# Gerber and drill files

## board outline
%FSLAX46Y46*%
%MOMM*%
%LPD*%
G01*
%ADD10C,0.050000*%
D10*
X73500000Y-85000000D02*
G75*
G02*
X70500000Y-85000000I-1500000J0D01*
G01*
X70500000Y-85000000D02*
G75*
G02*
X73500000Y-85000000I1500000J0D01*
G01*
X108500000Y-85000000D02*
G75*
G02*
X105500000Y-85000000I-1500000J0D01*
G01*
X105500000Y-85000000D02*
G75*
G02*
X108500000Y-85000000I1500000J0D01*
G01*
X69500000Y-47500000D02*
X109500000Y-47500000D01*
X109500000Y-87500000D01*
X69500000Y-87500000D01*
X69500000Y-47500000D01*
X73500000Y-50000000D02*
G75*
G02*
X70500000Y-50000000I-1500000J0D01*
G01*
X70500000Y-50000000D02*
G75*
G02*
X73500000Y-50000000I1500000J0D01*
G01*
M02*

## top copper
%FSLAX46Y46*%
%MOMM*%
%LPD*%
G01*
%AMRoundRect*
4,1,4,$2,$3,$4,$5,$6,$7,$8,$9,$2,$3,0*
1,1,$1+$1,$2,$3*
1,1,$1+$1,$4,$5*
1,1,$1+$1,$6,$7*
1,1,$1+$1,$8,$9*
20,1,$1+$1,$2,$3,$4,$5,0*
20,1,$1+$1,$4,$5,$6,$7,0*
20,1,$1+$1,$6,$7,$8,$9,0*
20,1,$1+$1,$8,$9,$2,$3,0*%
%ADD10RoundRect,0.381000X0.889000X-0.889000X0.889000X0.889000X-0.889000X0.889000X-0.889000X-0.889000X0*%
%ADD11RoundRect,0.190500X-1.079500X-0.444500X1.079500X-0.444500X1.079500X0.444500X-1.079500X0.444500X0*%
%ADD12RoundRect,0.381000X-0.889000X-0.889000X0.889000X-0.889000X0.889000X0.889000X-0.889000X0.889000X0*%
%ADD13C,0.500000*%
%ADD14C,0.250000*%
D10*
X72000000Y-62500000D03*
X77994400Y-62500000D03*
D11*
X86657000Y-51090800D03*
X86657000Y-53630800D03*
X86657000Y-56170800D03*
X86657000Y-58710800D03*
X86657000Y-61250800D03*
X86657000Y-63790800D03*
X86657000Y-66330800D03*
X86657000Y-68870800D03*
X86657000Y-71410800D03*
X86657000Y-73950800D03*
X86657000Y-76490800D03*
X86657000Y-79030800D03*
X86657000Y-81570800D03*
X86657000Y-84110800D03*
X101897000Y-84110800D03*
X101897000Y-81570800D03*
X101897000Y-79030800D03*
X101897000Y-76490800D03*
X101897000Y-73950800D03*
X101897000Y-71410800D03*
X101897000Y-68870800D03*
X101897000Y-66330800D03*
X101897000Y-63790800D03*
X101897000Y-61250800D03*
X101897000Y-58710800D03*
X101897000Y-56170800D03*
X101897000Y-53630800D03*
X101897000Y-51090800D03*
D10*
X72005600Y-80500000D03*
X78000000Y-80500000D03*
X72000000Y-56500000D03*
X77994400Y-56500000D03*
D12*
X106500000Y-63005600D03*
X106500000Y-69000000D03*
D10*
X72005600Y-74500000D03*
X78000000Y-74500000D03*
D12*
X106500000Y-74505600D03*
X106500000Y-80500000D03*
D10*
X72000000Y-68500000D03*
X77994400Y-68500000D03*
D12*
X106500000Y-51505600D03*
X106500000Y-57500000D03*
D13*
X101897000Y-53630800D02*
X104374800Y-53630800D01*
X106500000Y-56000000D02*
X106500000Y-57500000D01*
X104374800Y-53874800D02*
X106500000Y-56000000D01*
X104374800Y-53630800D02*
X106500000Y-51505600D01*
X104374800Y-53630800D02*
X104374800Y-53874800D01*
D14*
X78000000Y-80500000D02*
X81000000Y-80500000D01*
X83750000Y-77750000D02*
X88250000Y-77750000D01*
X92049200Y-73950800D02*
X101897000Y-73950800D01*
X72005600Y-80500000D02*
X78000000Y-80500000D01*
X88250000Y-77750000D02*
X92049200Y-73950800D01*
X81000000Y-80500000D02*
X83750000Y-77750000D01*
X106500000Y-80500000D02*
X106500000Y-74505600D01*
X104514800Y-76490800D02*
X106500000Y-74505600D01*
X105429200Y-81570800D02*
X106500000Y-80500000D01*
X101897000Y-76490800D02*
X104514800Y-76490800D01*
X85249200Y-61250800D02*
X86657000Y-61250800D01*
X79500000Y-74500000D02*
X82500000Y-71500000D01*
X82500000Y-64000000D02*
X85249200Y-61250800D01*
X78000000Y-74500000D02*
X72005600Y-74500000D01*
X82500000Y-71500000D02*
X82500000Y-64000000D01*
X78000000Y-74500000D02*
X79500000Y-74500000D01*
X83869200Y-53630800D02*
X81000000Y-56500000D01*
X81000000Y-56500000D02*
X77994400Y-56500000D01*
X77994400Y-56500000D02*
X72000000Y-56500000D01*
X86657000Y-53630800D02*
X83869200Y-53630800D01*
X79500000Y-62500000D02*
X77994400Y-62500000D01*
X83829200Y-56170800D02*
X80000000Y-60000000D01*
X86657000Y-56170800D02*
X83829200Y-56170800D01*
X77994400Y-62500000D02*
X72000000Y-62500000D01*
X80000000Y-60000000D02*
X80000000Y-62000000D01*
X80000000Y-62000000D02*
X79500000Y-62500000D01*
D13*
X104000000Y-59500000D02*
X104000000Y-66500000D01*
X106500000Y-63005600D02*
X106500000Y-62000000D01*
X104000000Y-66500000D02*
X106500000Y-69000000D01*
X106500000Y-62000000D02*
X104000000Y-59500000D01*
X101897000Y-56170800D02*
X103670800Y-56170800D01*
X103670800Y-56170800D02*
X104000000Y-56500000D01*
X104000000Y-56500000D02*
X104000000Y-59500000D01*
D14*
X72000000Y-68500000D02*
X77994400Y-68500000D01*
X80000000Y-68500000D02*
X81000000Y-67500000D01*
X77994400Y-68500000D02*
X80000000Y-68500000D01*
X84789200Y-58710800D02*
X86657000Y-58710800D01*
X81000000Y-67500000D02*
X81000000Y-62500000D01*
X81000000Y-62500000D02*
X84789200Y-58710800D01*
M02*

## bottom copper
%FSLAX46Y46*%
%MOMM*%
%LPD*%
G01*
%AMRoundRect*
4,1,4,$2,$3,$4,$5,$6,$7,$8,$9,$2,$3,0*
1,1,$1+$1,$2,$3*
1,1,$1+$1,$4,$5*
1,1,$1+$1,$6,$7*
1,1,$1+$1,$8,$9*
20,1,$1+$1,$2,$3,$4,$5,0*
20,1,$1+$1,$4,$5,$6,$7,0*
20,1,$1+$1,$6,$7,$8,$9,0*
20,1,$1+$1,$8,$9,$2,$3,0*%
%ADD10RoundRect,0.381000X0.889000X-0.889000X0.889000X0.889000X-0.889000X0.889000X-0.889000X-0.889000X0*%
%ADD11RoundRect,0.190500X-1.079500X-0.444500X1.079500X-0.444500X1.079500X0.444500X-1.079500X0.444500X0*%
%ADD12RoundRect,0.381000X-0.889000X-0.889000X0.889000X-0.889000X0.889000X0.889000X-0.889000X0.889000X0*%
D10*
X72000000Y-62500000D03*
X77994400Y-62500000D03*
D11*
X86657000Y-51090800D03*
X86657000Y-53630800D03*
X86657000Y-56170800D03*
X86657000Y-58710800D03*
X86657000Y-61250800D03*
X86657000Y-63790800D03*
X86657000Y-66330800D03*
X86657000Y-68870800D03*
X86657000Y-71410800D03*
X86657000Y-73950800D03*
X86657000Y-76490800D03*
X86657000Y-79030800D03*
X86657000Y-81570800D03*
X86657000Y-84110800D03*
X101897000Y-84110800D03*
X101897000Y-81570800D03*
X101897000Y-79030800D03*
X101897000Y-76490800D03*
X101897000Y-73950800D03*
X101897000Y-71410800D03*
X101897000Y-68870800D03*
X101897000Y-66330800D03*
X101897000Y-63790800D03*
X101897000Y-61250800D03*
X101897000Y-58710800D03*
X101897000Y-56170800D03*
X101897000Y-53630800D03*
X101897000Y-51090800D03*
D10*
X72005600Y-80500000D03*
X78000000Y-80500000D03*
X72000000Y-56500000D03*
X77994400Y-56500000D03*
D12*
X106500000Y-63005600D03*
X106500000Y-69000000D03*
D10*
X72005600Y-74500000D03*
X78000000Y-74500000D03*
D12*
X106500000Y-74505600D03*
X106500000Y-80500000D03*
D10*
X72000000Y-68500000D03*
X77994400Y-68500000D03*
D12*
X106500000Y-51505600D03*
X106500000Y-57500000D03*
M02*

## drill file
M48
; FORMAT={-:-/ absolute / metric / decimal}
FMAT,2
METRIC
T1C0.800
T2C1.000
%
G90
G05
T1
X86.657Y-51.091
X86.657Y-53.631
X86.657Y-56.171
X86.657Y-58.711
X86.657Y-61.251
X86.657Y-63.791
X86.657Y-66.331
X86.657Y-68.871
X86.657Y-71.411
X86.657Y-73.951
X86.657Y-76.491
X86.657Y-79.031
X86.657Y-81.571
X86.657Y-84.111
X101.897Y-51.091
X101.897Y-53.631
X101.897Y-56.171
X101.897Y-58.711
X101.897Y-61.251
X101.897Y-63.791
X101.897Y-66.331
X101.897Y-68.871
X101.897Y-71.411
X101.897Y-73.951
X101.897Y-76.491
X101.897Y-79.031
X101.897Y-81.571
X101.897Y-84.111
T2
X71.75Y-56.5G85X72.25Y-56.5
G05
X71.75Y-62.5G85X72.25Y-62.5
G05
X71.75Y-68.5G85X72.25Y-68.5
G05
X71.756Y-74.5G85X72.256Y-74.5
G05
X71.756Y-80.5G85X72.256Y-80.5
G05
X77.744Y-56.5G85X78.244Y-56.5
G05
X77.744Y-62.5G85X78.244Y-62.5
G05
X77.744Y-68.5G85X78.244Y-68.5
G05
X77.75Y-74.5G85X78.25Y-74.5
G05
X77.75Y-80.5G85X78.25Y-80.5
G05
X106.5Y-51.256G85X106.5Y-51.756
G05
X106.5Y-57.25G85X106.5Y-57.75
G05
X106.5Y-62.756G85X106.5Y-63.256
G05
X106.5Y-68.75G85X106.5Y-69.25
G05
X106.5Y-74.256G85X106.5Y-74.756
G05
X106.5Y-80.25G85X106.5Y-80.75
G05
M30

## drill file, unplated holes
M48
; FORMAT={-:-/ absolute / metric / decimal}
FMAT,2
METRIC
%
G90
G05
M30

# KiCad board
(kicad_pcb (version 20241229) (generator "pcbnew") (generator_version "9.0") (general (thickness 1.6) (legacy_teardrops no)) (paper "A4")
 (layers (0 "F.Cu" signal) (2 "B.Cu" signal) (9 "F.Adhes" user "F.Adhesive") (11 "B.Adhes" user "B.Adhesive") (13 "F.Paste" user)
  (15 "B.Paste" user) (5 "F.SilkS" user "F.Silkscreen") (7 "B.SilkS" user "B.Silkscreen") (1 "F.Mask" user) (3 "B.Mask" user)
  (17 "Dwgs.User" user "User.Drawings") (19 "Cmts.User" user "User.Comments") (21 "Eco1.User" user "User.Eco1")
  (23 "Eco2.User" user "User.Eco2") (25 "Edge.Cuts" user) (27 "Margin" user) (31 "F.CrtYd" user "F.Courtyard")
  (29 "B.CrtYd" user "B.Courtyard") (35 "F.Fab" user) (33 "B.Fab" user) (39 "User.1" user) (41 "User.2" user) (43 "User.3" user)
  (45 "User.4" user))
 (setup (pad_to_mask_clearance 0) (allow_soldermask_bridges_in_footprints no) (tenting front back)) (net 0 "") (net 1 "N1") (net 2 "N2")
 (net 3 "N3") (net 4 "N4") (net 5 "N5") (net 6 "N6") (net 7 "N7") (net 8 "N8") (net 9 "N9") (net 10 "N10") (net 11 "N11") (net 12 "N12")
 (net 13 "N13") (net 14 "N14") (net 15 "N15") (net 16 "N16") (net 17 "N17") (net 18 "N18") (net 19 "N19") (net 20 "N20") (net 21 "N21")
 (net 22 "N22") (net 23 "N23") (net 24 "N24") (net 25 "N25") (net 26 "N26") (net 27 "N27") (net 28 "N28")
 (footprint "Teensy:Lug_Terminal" (layer "F.Cu") (at 75.2512 62.5 90)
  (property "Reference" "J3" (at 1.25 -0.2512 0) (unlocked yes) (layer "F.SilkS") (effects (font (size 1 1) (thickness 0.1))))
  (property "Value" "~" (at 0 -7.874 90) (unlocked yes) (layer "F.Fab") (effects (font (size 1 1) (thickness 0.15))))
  (pad "1" thru_hole roundrect (at 0 -3.2512 90) (size 2.54 2.54) (drill oval 1 1.5) (layers "*.Cu" "*.Mask") (remove_unused_layers no)
   (roundrect_rratio 0.15) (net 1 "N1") (thermal_bridge_angle 45))
  (pad "1" thru_hole roundrect (at 0 2.7432 90) (size 2.54 2.54) (drill oval 1 1.5) (layers "*.Cu" "*.Mask") (remove_unused_layers no)
   (roundrect_rratio 0.15) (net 1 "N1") (thermal_bridge_angle 45)))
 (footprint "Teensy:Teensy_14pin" (layer "F.Cu") (at 91.737 58.7108)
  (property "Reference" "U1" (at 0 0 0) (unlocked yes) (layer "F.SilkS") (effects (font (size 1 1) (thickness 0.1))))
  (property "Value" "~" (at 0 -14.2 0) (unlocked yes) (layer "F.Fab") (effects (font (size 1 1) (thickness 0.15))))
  (pad "1" thru_hole roundrect (at -5.08 -7.62) (size 2.54 1.27) (drill 0.8) (layers "*.Cu" "*.Mask") (remove_unused_layers no)
   (roundrect_rratio 0.15) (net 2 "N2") (thermal_bridge_angle 45))
  (pad "2" thru_hole roundrect (at -5.08 -5.08) (size 2.54 1.27) (drill 0.8) (layers "*.Cu" "*.Mask") (remove_unused_layers no)
   (roundrect_rratio 0.15) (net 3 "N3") (thermal_bridge_angle 45))
  (pad "3" thru_hole roundrect (at -5.08 -2.54) (size 2.54 1.27) (drill 0.8) (layers "*.Cu" "*.Mask") (remove_unused_layers no)
   (roundrect_rratio 0.15) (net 1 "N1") (thermal_bridge_angle 45))
  (pad "4" thru_hole roundrect (at -5.08 0) (size 2.54 1.27) (drill 0.8) (layers "*.Cu" "*.Mask") (remove_unused_layers no)
   (roundrect_rratio 0.15) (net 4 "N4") (thermal_bridge_angle 45))
  (pad "5" thru_hole roundrect (at -5.08 2.54) (size 2.54 1.27) (drill 0.8) (layers "*.Cu" "*.Mask") (remove_unused_layers no)
   (roundrect_rratio 0.15) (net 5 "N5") (thermal_bridge_angle 45))
  (pad "6" thru_hole roundrect (at -5.08 5.08) (size 2.54 1.27) (drill 0.8) (layers "*.Cu" "*.Mask") (remove_unused_layers no)
   (roundrect_rratio 0.15) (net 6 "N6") (thermal_bridge_angle 45))
  (pad "7" thru_hole roundrect (at -5.08 7.62) (size 2.54 1.27) (drill 0.8) (layers "*.Cu" "*.Mask") (remove_unused_layers no)
   (roundrect_rratio 0.15) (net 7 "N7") (thermal_bridge_angle 45))
  (pad "8" thru_hole roundrect (at -5.08 10.16) (size 2.54 1.27) (drill 0.8) (layers "*.Cu" "*.Mask") (remove_unused_layers no)
   (roundrect_rratio 0.15) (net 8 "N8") (thermal_bridge_angle 45))
  (pad "9" thru_hole roundrect (at -5.08 12.7) (size 2.54 1.27) (drill 0.8) (layers "*.Cu" "*.Mask") (remove_unused_layers no)
   (roundrect_rratio 0.15) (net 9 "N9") (thermal_bridge_angle 45))
  (pad "10" thru_hole roundrect (at -5.08 15.24) (size 2.54 1.27) (drill 0.8) (layers "*.Cu" "*.Mask") (remove_unused_layers no)
   (roundrect_rratio 0.15) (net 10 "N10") (thermal_bridge_angle 45))
  (pad "11" thru_hole roundrect (at -5.08 17.78) (size 2.54 1.27) (drill 0.8) (layers "*.Cu" "*.Mask") (remove_unused_layers no)
   (roundrect_rratio 0.15) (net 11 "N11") (thermal_bridge_angle 45))
  (pad "12" thru_hole roundrect (at -5.08 20.32) (size 2.54 1.27) (drill 0.8) (layers "*.Cu" "*.Mask") (remove_unused_layers no)
   (roundrect_rratio 0.15) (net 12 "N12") (thermal_bridge_angle 45))
  (pad "13" thru_hole roundrect (at -5.08 22.86) (size 2.54 1.27) (drill 0.8) (layers "*.Cu" "*.Mask") (remove_unused_layers no)
   (roundrect_rratio 0.15) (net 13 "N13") (thermal_bridge_angle 45))
  (pad "14" thru_hole roundrect (at -5.08 25.4) (size 2.54 1.27) (drill 0.8) (layers "*.Cu" "*.Mask") (remove_unused_layers no)
   (roundrect_rratio 0.15) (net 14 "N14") (thermal_bridge_angle 45))
  (pad "15" thru_hole roundrect (at 10.16 25.4) (size 2.54 1.27) (drill 0.8) (layers "*.Cu" "*.Mask") (remove_unused_layers no)
   (roundrect_rratio 0.15) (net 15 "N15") (thermal_bridge_angle 45))
  (pad "16" thru_hole roundrect (at 10.16 22.86) (size 2.54 1.27) (drill 0.8) (layers "*.Cu" "*.Mask") (remove_unused_layers no)
   (roundrect_rratio 0.15) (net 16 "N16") (thermal_bridge_angle 45))
  (pad "17" thru_hole roundrect (at 10.16 20.32) (size 2.54 1.27) (drill 0.8) (layers "*.Cu" "*.Mask") (remove_unused_layers no)
   (roundrect_rratio 0.15) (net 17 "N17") (thermal_bridge_angle 45))
  (pad "18" thru_hole roundrect (at 10.16 17.78) (size 2.54 1.27) (drill 0.8) (layers "*.Cu" "*.Mask") (remove_unused_layers no)
   (roundrect_rratio 0.15) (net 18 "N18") (thermal_bridge_angle 45))
  (pad "19" thru_hole roundrect (at 10.16 15.24) (size 2.54 1.27) (drill 0.8) (layers "*.Cu" "*.Mask") (remove_unused_layers no)
   (roundrect_rratio 0.15) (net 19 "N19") (thermal_bridge_angle 45))
  (pad "20" thru_hole roundrect (at 10.16 12.7) (size 2.54 1.27) (drill 0.8) (layers "*.Cu" "*.Mask") (remove_unused_layers no)
   (roundrect_rratio 0.15) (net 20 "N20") (thermal_bridge_angle 45))
  (pad "21" thru_hole roundrect (at 10.16 10.16) (size 2.54 1.27) (drill 0.8) (layers "*.Cu" "*.Mask") (remove_unused_layers no)
   (roundrect_rratio 0.15) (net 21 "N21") (thermal_bridge_angle 45))
  (pad "22" thru_hole roundrect (at 10.16 7.62) (size 2.54 1.27) (drill 0.8) (layers "*.Cu" "*.Mask") (remove_unused_layers no)
   (roundrect_rratio 0.15) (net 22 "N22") (thermal_bridge_angle 45))
  (pad "23" thru_hole roundrect (at 10.16 5.08) (size 2.54 1.27) (drill 0.8) (layers "*.Cu" "*.Mask") (remove_unused_layers no)
   (roundrect_rratio 0.15) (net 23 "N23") (thermal_bridge_angle 45))
  (pad "24" thru_hole roundrect (at 10.16 2.54) (size 2.54 1.27) (drill 0.8) (layers "*.Cu" "*.Mask") (remove_unused_layers no)
   (roundrect_rratio 0.15) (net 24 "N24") (thermal_bridge_angle 45))
  (pad "25" thru_hole roundrect (at 10.16 0) (size 2.54 1.27) (drill 0.8) (layers "*.Cu" "*.Mask") (remove_unused_layers no)
   (roundrect_rratio 0.15) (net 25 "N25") (thermal_bridge_angle 45))
  (pad "26" thru_hole roundrect (at 10.16 -2.54) (size 2.54 1.27) (drill 0.8) (layers "*.Cu" "*.Mask") (remove_unused_layers no)
   (roundrect_rratio 0.15) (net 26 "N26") (thermal_bridge_angle 45))
  (pad "27" thru_hole roundrect (at 10.16 -5.08) (size 2.54 1.27) (drill 0.8) (layers "*.Cu" "*.Mask") (remove_unused_layers no)
   (roundrect_rratio 0.15) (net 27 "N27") (thermal_bridge_angle 45))
  (pad "28" thru_hole roundrect (at 10.16 -7.62) (size 2.54 1.27) (drill 0.8) (layers "*.Cu" "*.Mask") (remove_unused_layers no)
   (roundrect_rratio 0.15) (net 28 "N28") (thermal_bridge_angle 45)))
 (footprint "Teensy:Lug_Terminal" (layer "F.Cu") (at 75.2568 80.5 90)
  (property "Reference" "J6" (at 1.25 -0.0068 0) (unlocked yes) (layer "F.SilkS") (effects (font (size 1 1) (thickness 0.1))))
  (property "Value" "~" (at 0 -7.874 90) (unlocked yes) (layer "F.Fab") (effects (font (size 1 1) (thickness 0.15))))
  (pad "1" thru_hole roundrect (at 0 -3.2512 90) (size 2.54 2.54) (drill oval 1 1.5) (layers "*.Cu" "*.Mask") (remove_unused_layers no)
   (roundrect_rratio 0.15) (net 19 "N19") (thermal_bridge_angle 45))
  (pad "1" thru_hole roundrect (at 0 2.7432 90) (size 2.54 2.54) (drill oval 1 1.5) (layers "*.Cu" "*.Mask") (remove_unused_layers no)
   (roundrect_rratio 0.15) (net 19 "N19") (thermal_bridge_angle 45)))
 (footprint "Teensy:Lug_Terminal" (layer "F.Cu") (at 75.2512 56.5 90)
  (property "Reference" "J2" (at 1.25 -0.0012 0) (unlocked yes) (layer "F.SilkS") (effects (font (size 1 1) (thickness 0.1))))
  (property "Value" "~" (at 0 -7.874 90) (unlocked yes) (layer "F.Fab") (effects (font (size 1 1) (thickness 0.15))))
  (pad "1" thru_hole roundrect (at 0 -3.2512 90) (size 2.54 2.54) (drill oval 1 1.5) (layers "*.Cu" "*.Mask") (remove_unused_layers no)
   (roundrect_rratio 0.15) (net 3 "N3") (thermal_bridge_angle 45))
  (pad "1" thru_hole roundrect (at 0 2.7432 90) (size 2.54 2.54) (drill oval 1 1.5) (layers "*.Cu" "*.Mask") (remove_unused_layers no)
   (roundrect_rratio 0.15) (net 3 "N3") (thermal_bridge_angle 45)))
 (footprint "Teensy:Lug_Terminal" (layer "F.Cu") (at 106.5 66.2568)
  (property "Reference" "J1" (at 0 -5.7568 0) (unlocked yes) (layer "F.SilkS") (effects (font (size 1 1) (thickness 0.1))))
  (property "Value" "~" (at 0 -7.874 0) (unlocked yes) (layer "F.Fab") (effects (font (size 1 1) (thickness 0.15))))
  (pad "1" thru_hole roundrect (at 0 -3.2512) (size 2.54 2.54) (drill oval 1 1.5) (layers "*.Cu" "*.Mask") (remove_unused_layers no)
   (roundrect_rratio 0.15) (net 26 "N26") (thermal_bridge_angle 45))
  (pad "1" thru_hole roundrect (at 0 2.7432) (size 2.54 2.54) (drill oval 1 1.5) (layers "*.Cu" "*.Mask") (remove_unused_layers no)
   (roundrect_rratio 0.15) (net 26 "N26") (thermal_bridge_angle 45)))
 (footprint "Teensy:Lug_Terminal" (layer "F.Cu") (at 75.2568 74.5 90)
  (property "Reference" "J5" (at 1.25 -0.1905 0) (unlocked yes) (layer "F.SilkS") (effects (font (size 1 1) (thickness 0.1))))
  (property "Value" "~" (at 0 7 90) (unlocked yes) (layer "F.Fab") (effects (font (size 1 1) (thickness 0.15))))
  (pad "1" thru_hole roundrect (at 0 -3.2512 90) (size 2.54 2.54) (drill oval 1 1.5) (layers "*.Cu" "*.Mask") (remove_unused_layers no)
   (roundrect_rratio 0.15) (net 5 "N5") (thermal_bridge_angle 45))
  (pad "1" thru_hole roundrect (at 0 2.7432 90) (size 2.54 2.54) (drill oval 1 1.5) (layers "*.Cu" "*.Mask") (remove_unused_layers no)
   (roundrect_rratio 0.15) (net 5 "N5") (thermal_bridge_angle 45)))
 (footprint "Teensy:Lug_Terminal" (layer "F.Cu") (at 106.5 77.7568)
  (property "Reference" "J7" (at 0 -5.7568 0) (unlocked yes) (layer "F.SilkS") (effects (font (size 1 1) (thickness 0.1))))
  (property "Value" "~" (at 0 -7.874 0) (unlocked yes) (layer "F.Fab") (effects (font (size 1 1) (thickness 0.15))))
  (pad "1" thru_hole roundrect (at 0 -3.2512) (size 2.54 2.54) (drill oval 1 1.5) (layers "*.Cu" "*.Mask") (remove_unused_layers no)
   (roundrect_rratio 0.15) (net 18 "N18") (thermal_bridge_angle 45))
  (pad "1" thru_hole roundrect (at 0 2.7432) (size 2.54 2.54) (drill oval 1 1.5) (layers "*.Cu" "*.Mask") (remove_unused_layers no)
   (roundrect_rratio 0.15) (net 18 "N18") (thermal_bridge_angle 45)))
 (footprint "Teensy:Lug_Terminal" (layer "F.Cu") (at 75.2512 68.5 90)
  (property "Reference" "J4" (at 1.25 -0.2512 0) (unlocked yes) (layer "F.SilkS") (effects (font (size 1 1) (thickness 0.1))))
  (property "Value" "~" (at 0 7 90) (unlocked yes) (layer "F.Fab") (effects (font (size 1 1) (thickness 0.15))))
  (pad "1" thru_hole roundrect (at 0 -3.2512 90) (size 2.54 2.54) (drill oval 1 1.5) (layers "*.Cu" "*.Mask") (remove_unused_layers no)
   (roundrect_rratio 0.15) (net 4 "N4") (thermal_bridge_angle 45))
  (pad "1" thru_hole roundrect (at 0 2.7432 90) (size 2.54 2.54) (drill oval 1 1.5) (layers "*.Cu" "*.Mask") (remove_unused_layers no)
   (roundrect_rratio 0.15) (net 4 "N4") (thermal_bridge_angle 45)))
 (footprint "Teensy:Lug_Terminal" (layer "F.Cu") (at 106.5 54.7568)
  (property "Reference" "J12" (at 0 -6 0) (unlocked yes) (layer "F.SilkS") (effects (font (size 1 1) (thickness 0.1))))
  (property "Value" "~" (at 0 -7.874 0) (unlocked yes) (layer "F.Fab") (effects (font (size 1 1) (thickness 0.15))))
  (pad "1" thru_hole roundrect (at 0 -3.2512) (size 2.54 2.54) (drill oval 1 1.5) (layers "*.Cu" "*.Mask") (remove_unused_layers no)
   (roundrect_rratio 0.15) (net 27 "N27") (thermal_bridge_angle 45))
  (pad "1" thru_hole roundrect (at 0 2.7432) (size 2.54 2.54) (drill oval 1 1.5) (layers "*.Cu" "*.Mask") (remove_unused_layers no)
   (roundrect_rratio 0.15) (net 27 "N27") (thermal_bridge_angle 45)))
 (gr_circle (center 72 85) (end 73.5 85) (stroke (width 0.05) (type default)) (fill no) (layer "Edge.Cuts"))
 (gr_circle (center 107 85) (end 108.5 85) (stroke (width 0.05) (type default)) (fill no) (layer "Edge.Cuts"))
 (gr_rect (start 69.5 47.5) (end 109.5 87.5) (stroke (width 0.05) (type solid)) (fill no) (layer "Edge.Cuts"))
 (gr_circle (center 72 50) (end 73.5 50) (stroke (width 0.05) (type default)) (fill no) (layer "Edge.Cuts"))
 (segment (start 101.897 53.6308) (end 104.3748 53.6308) (width 0.5) (layer "F.Cu") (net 27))
 (segment (start 106.5 56) (end 106.5 57.5) (width 0.5) (layer "F.Cu") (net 27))
 (segment (start 104.3748 53.8748) (end 106.5 56) (width 0.5) (layer "F.Cu") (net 27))
 (segment (start 104.3748 53.6308) (end 106.5 51.5056) (width 0.5) (layer "F.Cu") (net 27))
 (segment (start 104.3748 53.6308) (end 104.3748 53.8748) (width 0.5) (layer "F.Cu") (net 27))
 (segment (start 78 80.5) (end 81 80.5) (width 0.25) (layer "F.Cu") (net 19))
 (segment (start 83.75 77.75) (end 88.25 77.75) (width 0.25) (layer "F.Cu") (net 19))
 (segment (start 92.0492 73.9508) (end 101.897 73.9508) (width 0.25) (layer "F.Cu") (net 19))
 (segment (start 72.0056 80.5) (end 78 80.5) (width 0.25) (layer "F.Cu") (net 19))
 (segment (start 88.25 77.75) (end 92.0492 73.9508) (width 0.25) (layer "F.Cu") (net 19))
 (segment (start 81 80.5) (end 83.75 77.75) (width 0.25) (layer "F.Cu") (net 19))
 (segment (start 106.5 80.5) (end 106.5 74.5056) (width 0.25) (layer "F.Cu") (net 18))
 (segment (start 104.5148 76.4908) (end 106.5 74.5056) (width 0.25) (layer "F.Cu") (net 18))
 (segment (start 105.4292 81.5708) (end 106.5 80.5) (width 0.25) (layer "F.Cu") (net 18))
 (segment (start 101.897 76.4908) (end 104.5148 76.4908) (width 0.25) (layer "F.Cu") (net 18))
 (segment (start 85.2492 61.2508) (end 86.657 61.2508) (width 0.25) (layer "F.Cu") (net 5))
 (segment (start 79.5 74.5) (end 82.5 71.5) (width 0.25) (layer "F.Cu") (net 5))
 (segment (start 82.5 64) (end 85.2492 61.2508) (width 0.25) (layer "F.Cu") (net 5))
 (segment (start 78 74.5) (end 72.0056 74.5) (width 0.25) (layer "F.Cu") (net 5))
 (segment (start 82.5 71.5) (end 82.5 64) (width 0.25) (layer "F.Cu") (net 5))
 (segment (start 78 74.5) (end 79.5 74.5) (width 0.25) (layer "F.Cu") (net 5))
 (segment (start 83.8692 53.6308) (end 81 56.5) (width 0.25) (layer "F.Cu") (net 3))
 (segment (start 81 56.5) (end 77.9944 56.5) (width 0.25) (layer "F.Cu") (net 3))
 (segment (start 77.9944 56.5) (end 72 56.5) (width 0.25) (layer "F.Cu") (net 3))
 (segment (start 86.657 53.6308) (end 83.8692 53.6308) (width 0.25) (layer "F.Cu") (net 3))
 (segment (start 79.5 62.5) (end 77.9944 62.5) (width 0.25) (layer "F.Cu") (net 1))
 (segment (start 83.8292 56.1708) (end 80 60) (width 0.25) (layer "F.Cu") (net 1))
 (segment (start 86.657 56.1708) (end 83.8292 56.1708) (width 0.25) (layer "F.Cu") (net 1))
 (segment (start 77.9944 62.5) (end 72 62.5) (width 0.25) (layer "F.Cu") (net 1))
 (segment (start 80 60) (end 80 62) (width 0.25) (layer "F.Cu") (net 1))
 (segment (start 80 62) (end 79.5 62.5) (width 0.25) (layer "F.Cu") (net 1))
 (segment (start 104 59.5) (end 104 66.5) (width 0.5) (layer "F.Cu") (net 26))
 (segment (start 106.5 63.0056) (end 106.5 62) (width 0.5) (layer "F.Cu") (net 26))
 (segment (start 104 66.5) (end 106.5 69) (width 0.5) (layer "F.Cu") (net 26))
 (segment (start 106.5 62) (end 104 59.5) (width 0.5) (layer "F.Cu") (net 26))
 (segment (start 101.897 56.1708) (end 103.6708 56.1708) (width 0.5) (layer "F.Cu") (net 26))
 (segment (start 103.6708 56.1708) (end 104 56.5) (width 0.5) (layer "F.Cu") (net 26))
 (segment (start 104 56.5) (end 104 59.5) (width 0.5) (layer "F.Cu") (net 26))
 (segment (start 72 68.5) (end 77.9944 68.5) (width 0.25) (layer "F.Cu") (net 4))
 (segment (start 80 68.5) (end 81 67.5) (width 0.25) (layer "F.Cu") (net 4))
 (segment (start 77.9944 68.5) (end 80 68.5) (width 0.25) (layer "F.Cu") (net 4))
 (segment (start 84.7892 58.7108) (end 86.657 58.7108) (width 0.25) (layer "F.Cu") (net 4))
 (segment (start 81 67.5) (end 81 62.5) (width 0.25) (layer "F.Cu") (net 4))
 (segment (start 81 62.5) (end 84.7892 58.7108) (width 0.25) (layer "F.Cu") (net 4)))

